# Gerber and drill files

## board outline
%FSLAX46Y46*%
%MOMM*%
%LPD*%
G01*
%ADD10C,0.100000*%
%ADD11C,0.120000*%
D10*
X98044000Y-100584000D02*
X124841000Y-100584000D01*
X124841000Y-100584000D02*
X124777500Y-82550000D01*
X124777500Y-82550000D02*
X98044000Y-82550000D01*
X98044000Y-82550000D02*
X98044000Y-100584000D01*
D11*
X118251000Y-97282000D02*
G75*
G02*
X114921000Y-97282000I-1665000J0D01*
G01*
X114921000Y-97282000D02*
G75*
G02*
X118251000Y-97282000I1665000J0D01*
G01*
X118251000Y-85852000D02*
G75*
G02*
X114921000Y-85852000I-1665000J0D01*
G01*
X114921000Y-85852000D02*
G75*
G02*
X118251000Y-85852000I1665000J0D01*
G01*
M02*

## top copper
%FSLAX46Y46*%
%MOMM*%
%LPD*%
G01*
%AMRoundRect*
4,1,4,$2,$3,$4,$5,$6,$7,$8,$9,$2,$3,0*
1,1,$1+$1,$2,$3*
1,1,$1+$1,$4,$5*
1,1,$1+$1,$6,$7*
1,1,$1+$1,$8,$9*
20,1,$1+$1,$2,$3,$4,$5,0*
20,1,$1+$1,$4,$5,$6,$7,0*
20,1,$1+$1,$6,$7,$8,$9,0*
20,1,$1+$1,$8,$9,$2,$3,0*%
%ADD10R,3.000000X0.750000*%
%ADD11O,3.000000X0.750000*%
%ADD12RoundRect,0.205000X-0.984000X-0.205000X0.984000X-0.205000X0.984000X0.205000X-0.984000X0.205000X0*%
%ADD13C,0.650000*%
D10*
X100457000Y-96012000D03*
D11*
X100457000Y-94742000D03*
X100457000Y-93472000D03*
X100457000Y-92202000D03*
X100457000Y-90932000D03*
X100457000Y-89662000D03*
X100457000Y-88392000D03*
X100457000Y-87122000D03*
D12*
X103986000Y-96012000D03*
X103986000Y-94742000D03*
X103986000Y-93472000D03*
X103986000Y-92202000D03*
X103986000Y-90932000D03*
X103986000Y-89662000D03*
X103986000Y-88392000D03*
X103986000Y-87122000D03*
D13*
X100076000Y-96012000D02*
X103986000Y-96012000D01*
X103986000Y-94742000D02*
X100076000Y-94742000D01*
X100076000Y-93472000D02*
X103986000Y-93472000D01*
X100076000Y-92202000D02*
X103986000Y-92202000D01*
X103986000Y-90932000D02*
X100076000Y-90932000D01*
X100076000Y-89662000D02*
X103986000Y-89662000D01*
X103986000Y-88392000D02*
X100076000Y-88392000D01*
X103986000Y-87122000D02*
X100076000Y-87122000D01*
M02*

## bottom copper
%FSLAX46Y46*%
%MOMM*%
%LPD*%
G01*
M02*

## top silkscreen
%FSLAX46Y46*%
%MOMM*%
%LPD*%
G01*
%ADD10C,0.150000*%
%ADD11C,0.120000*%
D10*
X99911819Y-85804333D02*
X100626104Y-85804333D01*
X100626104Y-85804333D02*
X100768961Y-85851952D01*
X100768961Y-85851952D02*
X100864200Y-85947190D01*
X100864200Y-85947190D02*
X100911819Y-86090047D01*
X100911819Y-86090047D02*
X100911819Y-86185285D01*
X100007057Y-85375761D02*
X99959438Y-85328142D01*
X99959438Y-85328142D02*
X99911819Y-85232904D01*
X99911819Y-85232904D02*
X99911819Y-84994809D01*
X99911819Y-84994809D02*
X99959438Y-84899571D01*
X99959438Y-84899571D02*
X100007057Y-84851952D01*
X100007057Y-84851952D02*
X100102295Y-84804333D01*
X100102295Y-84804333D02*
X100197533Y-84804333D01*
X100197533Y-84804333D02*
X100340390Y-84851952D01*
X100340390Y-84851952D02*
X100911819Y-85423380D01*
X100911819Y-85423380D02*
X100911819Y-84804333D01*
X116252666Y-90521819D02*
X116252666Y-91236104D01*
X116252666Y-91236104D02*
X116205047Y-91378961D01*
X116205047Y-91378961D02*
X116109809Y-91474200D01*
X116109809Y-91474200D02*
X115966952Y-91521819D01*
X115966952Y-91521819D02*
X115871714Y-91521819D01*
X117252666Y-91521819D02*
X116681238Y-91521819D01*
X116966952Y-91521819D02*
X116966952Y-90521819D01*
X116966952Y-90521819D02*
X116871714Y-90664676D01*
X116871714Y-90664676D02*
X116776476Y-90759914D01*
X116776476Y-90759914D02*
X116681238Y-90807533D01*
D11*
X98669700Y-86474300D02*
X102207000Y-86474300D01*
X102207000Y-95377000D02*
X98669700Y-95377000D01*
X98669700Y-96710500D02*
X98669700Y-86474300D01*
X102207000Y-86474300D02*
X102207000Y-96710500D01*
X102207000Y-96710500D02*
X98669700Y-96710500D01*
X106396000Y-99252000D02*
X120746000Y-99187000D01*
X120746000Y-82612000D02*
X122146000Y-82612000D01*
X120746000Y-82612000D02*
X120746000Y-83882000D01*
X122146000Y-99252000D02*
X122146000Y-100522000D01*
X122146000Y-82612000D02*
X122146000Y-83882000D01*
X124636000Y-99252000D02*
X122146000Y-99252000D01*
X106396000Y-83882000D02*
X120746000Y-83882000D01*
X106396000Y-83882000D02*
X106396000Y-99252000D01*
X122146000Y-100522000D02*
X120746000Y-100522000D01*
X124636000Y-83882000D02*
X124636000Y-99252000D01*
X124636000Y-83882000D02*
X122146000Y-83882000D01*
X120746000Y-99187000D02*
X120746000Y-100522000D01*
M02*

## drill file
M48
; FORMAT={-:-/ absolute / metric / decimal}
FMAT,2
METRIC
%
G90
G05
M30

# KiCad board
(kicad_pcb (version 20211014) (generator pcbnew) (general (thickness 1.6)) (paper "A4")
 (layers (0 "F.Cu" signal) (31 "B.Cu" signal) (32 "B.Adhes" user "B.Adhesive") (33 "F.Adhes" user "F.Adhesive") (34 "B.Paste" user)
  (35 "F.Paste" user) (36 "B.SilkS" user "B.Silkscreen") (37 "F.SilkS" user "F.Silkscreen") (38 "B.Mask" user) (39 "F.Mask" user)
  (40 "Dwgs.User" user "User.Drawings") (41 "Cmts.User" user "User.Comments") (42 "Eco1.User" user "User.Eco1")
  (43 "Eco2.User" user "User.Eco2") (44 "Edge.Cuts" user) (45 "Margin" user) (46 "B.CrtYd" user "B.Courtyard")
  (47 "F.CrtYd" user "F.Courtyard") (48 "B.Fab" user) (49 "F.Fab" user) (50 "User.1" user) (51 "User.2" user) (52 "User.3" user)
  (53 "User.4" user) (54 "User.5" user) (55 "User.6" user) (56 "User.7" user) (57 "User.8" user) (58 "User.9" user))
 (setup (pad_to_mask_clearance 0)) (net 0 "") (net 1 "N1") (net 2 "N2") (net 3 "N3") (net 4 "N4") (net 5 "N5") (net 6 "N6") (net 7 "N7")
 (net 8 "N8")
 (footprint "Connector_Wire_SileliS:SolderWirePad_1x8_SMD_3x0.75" (layer "F.Cu") (at 97.4697 91.5543 90)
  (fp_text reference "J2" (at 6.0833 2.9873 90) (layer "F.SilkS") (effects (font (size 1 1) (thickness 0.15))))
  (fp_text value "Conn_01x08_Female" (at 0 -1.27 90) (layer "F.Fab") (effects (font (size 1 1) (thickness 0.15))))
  (fp_line (start 5.08 1.2) (end 5.08 4.7373) (layer "F.SilkS") (width 0.12))
  (fp_line (start -3.8227 4.7373) (end -3.8227 1.2) (layer "F.SilkS") (width 0.12))
  (fp_line (start -5.1562 1.2) (end 5.08 1.2) (layer "F.SilkS") (width 0.12))
  (fp_line (start 5.08 4.7373) (end -5.1562 4.7373) (layer "F.SilkS") (width 0.12))
  (fp_line (start -5.1562 4.7373) (end -5.1562 1.2) (layer "F.SilkS") (width 0.12))
  (pad "1" smd rect locked (at -4.4577 2.9873 90) (size 0.75 3) (layers "F.Cu" "F.Mask") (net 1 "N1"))
  (pad "2" smd oval locked (at -3.1877 2.9873 90) (size 0.75 3) (layers "F.Cu" "F.Mask") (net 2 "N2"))
  (pad "3" smd oval locked (at -1.9177 2.9873 90) (size 0.75 3) (layers "F.Cu" "F.Mask") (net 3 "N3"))
  (pad "4" smd oval locked (at -0.6477 2.9873 90) (size 0.75 3) (layers "F.Cu" "F.Mask") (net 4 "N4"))
  (pad "5" smd oval locked (at 0.6223 2.9873 90) (size 0.75 3) (layers "F.Cu" "F.Mask") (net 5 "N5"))
  (pad "6" smd oval locked (at 1.8923 2.9873 90) (size 0.75 3) (layers "F.Cu" "F.Mask") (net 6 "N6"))
  (pad "7" smd oval locked (at 3.1623 2.9873 90) (size 0.75 3) (layers "F.Cu" "F.Mask") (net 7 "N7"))
  (pad "8" smd oval locked (at 4.4323 2.9873 90) (size 0.75 3) (layers "F.Cu" "F.Mask") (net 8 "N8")))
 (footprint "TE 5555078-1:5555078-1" (layer "F.Cu") (at 116.586 91.567)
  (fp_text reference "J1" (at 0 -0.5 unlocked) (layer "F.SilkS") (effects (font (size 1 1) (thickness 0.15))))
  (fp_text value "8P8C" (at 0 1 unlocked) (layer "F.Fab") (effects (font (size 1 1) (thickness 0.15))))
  (fp_line (start -10.19 7.685) (end 4.16 7.62) (layer "F.SilkS") (width 0.12))
  (fp_line (start 4.16 -8.955) (end 5.56 -8.955) (layer "F.SilkS") (width 0.12))
  (fp_line (start 4.16 -8.955) (end 4.16 -7.685) (layer "F.SilkS") (width 0.12))
  (fp_line (start 5.56 7.685) (end 5.56 8.955) (layer "F.SilkS") (width 0.12))
  (fp_line (start 5.56 -8.955) (end 5.56 -7.685) (layer "F.SilkS") (width 0.12))
  (fp_line (start 8.05 7.685) (end 5.56 7.685) (layer "F.SilkS") (width 0.12))
  (fp_line (start -10.19 -7.685) (end 4.16 -7.685) (layer "F.SilkS") (width 0.12))
  (fp_line (start -10.19 -7.685) (end -10.19 7.685) (layer "F.SilkS") (width 0.12))
  (fp_line (start 5.56 8.955) (end 4.16 8.955) (layer "F.SilkS") (width 0.12))
  (fp_line (start 8.05 -7.685) (end 8.05 7.685) (layer "F.SilkS") (width 0.12))
  (fp_line (start 8.05 -7.685) (end 5.56 -7.685) (layer "F.SilkS") (width 0.12))
  (fp_line (start 4.16 7.62) (end 4.16 8.955) (layer "F.SilkS") (width 0.12))
  (fp_circle (center 0 5.715) (end 1.665 5.715) (layer "Edge.Cuts") (width 0.12) (fill none))
  (fp_circle (center 0 -5.715) (end 1.665 -5.715) (layer "Edge.Cuts") (width 0.12) (fill none))
  (pad "1" smd roundrect (at -12.6 4.445) (size 2.378 0.82) (layers "F.Cu" "F.Paste" "F.Mask") (roundrect_rratio 0.25) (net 1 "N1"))
  (pad "2" smd roundrect (at -12.6 3.175) (size 2.378 0.82) (layers "F.Cu" "F.Paste" "F.Mask") (roundrect_rratio 0.25) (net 2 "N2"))
  (pad "3" smd roundrect (at -12.6 1.905) (size 2.378 0.82) (layers "F.Cu" "F.Paste" "F.Mask") (roundrect_rratio 0.25) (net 3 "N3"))
  (pad "4" smd roundrect (at -12.6 0.635) (size 2.378 0.82) (layers "F.Cu" "F.Paste" "F.Mask") (roundrect_rratio 0.25) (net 4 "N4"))
  (pad "5" smd roundrect (at -12.6 -0.635) (size 2.378 0.82) (layers "F.Cu" "F.Paste" "F.Mask") (roundrect_rratio 0.25) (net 5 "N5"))
  (pad "6" smd roundrect (at -12.6 -1.905) (size 2.378 0.82) (layers "F.Cu" "F.Paste" "F.Mask") (roundrect_rratio 0.25) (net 6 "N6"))
  (pad "7" smd roundrect (at -12.6 -3.175) (size 2.378 0.82) (layers "F.Cu" "F.Paste" "F.Mask") (roundrect_rratio 0.25) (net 7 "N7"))
  (pad "8" smd roundrect (at -12.6 -4.445) (size 2.378 0.82) (layers "F.Cu" "F.Paste" "F.Mask") (roundrect_rratio 0.25) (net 8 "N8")))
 (gr_line (start 98.044 100.584) (end 124.841 100.584) (layer "Edge.Cuts") (width 0.1))
 (gr_line (start 124.841 100.584) (end 124.7775 82.55) (layer "Edge.Cuts") (width 0.1))
 (gr_line (start 124.7775 82.55) (end 98.044 82.55) (layer "Edge.Cuts") (width 0.1))
 (gr_line (start 98.044 82.55) (end 98.044 100.584) (layer "Edge.Cuts") (width 0.1))
 (segment (start 100.076 96.012) (end 103.986 96.012) (width 0.65) (layer "F.Cu") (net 1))
 (segment (start 103.986 94.742) (end 100.076 94.742) (width 0.65) (layer "F.Cu") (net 2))
 (segment (start 100.076 93.472) (end 103.986 93.472) (width 0.65) (layer "F.Cu") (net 3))
 (segment (start 100.076 92.202) (end 103.986 92.202) (width 0.65) (layer "F.Cu") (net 4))
 (segment (start 103.986 90.932) (end 100.076 90.932) (width 0.65) (layer "F.Cu") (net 5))
 (segment (start 100.076 89.662) (end 103.986 89.662) (width 0.65) (layer "F.Cu") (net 6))
 (segment (start 103.986 88.392) (end 100.076 88.392) (width 0.65) (layer "F.Cu") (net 7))
 (segment (start 103.986 87.122) (end 100.076 87.122) (width 0.65) (layer "F.Cu") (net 8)))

